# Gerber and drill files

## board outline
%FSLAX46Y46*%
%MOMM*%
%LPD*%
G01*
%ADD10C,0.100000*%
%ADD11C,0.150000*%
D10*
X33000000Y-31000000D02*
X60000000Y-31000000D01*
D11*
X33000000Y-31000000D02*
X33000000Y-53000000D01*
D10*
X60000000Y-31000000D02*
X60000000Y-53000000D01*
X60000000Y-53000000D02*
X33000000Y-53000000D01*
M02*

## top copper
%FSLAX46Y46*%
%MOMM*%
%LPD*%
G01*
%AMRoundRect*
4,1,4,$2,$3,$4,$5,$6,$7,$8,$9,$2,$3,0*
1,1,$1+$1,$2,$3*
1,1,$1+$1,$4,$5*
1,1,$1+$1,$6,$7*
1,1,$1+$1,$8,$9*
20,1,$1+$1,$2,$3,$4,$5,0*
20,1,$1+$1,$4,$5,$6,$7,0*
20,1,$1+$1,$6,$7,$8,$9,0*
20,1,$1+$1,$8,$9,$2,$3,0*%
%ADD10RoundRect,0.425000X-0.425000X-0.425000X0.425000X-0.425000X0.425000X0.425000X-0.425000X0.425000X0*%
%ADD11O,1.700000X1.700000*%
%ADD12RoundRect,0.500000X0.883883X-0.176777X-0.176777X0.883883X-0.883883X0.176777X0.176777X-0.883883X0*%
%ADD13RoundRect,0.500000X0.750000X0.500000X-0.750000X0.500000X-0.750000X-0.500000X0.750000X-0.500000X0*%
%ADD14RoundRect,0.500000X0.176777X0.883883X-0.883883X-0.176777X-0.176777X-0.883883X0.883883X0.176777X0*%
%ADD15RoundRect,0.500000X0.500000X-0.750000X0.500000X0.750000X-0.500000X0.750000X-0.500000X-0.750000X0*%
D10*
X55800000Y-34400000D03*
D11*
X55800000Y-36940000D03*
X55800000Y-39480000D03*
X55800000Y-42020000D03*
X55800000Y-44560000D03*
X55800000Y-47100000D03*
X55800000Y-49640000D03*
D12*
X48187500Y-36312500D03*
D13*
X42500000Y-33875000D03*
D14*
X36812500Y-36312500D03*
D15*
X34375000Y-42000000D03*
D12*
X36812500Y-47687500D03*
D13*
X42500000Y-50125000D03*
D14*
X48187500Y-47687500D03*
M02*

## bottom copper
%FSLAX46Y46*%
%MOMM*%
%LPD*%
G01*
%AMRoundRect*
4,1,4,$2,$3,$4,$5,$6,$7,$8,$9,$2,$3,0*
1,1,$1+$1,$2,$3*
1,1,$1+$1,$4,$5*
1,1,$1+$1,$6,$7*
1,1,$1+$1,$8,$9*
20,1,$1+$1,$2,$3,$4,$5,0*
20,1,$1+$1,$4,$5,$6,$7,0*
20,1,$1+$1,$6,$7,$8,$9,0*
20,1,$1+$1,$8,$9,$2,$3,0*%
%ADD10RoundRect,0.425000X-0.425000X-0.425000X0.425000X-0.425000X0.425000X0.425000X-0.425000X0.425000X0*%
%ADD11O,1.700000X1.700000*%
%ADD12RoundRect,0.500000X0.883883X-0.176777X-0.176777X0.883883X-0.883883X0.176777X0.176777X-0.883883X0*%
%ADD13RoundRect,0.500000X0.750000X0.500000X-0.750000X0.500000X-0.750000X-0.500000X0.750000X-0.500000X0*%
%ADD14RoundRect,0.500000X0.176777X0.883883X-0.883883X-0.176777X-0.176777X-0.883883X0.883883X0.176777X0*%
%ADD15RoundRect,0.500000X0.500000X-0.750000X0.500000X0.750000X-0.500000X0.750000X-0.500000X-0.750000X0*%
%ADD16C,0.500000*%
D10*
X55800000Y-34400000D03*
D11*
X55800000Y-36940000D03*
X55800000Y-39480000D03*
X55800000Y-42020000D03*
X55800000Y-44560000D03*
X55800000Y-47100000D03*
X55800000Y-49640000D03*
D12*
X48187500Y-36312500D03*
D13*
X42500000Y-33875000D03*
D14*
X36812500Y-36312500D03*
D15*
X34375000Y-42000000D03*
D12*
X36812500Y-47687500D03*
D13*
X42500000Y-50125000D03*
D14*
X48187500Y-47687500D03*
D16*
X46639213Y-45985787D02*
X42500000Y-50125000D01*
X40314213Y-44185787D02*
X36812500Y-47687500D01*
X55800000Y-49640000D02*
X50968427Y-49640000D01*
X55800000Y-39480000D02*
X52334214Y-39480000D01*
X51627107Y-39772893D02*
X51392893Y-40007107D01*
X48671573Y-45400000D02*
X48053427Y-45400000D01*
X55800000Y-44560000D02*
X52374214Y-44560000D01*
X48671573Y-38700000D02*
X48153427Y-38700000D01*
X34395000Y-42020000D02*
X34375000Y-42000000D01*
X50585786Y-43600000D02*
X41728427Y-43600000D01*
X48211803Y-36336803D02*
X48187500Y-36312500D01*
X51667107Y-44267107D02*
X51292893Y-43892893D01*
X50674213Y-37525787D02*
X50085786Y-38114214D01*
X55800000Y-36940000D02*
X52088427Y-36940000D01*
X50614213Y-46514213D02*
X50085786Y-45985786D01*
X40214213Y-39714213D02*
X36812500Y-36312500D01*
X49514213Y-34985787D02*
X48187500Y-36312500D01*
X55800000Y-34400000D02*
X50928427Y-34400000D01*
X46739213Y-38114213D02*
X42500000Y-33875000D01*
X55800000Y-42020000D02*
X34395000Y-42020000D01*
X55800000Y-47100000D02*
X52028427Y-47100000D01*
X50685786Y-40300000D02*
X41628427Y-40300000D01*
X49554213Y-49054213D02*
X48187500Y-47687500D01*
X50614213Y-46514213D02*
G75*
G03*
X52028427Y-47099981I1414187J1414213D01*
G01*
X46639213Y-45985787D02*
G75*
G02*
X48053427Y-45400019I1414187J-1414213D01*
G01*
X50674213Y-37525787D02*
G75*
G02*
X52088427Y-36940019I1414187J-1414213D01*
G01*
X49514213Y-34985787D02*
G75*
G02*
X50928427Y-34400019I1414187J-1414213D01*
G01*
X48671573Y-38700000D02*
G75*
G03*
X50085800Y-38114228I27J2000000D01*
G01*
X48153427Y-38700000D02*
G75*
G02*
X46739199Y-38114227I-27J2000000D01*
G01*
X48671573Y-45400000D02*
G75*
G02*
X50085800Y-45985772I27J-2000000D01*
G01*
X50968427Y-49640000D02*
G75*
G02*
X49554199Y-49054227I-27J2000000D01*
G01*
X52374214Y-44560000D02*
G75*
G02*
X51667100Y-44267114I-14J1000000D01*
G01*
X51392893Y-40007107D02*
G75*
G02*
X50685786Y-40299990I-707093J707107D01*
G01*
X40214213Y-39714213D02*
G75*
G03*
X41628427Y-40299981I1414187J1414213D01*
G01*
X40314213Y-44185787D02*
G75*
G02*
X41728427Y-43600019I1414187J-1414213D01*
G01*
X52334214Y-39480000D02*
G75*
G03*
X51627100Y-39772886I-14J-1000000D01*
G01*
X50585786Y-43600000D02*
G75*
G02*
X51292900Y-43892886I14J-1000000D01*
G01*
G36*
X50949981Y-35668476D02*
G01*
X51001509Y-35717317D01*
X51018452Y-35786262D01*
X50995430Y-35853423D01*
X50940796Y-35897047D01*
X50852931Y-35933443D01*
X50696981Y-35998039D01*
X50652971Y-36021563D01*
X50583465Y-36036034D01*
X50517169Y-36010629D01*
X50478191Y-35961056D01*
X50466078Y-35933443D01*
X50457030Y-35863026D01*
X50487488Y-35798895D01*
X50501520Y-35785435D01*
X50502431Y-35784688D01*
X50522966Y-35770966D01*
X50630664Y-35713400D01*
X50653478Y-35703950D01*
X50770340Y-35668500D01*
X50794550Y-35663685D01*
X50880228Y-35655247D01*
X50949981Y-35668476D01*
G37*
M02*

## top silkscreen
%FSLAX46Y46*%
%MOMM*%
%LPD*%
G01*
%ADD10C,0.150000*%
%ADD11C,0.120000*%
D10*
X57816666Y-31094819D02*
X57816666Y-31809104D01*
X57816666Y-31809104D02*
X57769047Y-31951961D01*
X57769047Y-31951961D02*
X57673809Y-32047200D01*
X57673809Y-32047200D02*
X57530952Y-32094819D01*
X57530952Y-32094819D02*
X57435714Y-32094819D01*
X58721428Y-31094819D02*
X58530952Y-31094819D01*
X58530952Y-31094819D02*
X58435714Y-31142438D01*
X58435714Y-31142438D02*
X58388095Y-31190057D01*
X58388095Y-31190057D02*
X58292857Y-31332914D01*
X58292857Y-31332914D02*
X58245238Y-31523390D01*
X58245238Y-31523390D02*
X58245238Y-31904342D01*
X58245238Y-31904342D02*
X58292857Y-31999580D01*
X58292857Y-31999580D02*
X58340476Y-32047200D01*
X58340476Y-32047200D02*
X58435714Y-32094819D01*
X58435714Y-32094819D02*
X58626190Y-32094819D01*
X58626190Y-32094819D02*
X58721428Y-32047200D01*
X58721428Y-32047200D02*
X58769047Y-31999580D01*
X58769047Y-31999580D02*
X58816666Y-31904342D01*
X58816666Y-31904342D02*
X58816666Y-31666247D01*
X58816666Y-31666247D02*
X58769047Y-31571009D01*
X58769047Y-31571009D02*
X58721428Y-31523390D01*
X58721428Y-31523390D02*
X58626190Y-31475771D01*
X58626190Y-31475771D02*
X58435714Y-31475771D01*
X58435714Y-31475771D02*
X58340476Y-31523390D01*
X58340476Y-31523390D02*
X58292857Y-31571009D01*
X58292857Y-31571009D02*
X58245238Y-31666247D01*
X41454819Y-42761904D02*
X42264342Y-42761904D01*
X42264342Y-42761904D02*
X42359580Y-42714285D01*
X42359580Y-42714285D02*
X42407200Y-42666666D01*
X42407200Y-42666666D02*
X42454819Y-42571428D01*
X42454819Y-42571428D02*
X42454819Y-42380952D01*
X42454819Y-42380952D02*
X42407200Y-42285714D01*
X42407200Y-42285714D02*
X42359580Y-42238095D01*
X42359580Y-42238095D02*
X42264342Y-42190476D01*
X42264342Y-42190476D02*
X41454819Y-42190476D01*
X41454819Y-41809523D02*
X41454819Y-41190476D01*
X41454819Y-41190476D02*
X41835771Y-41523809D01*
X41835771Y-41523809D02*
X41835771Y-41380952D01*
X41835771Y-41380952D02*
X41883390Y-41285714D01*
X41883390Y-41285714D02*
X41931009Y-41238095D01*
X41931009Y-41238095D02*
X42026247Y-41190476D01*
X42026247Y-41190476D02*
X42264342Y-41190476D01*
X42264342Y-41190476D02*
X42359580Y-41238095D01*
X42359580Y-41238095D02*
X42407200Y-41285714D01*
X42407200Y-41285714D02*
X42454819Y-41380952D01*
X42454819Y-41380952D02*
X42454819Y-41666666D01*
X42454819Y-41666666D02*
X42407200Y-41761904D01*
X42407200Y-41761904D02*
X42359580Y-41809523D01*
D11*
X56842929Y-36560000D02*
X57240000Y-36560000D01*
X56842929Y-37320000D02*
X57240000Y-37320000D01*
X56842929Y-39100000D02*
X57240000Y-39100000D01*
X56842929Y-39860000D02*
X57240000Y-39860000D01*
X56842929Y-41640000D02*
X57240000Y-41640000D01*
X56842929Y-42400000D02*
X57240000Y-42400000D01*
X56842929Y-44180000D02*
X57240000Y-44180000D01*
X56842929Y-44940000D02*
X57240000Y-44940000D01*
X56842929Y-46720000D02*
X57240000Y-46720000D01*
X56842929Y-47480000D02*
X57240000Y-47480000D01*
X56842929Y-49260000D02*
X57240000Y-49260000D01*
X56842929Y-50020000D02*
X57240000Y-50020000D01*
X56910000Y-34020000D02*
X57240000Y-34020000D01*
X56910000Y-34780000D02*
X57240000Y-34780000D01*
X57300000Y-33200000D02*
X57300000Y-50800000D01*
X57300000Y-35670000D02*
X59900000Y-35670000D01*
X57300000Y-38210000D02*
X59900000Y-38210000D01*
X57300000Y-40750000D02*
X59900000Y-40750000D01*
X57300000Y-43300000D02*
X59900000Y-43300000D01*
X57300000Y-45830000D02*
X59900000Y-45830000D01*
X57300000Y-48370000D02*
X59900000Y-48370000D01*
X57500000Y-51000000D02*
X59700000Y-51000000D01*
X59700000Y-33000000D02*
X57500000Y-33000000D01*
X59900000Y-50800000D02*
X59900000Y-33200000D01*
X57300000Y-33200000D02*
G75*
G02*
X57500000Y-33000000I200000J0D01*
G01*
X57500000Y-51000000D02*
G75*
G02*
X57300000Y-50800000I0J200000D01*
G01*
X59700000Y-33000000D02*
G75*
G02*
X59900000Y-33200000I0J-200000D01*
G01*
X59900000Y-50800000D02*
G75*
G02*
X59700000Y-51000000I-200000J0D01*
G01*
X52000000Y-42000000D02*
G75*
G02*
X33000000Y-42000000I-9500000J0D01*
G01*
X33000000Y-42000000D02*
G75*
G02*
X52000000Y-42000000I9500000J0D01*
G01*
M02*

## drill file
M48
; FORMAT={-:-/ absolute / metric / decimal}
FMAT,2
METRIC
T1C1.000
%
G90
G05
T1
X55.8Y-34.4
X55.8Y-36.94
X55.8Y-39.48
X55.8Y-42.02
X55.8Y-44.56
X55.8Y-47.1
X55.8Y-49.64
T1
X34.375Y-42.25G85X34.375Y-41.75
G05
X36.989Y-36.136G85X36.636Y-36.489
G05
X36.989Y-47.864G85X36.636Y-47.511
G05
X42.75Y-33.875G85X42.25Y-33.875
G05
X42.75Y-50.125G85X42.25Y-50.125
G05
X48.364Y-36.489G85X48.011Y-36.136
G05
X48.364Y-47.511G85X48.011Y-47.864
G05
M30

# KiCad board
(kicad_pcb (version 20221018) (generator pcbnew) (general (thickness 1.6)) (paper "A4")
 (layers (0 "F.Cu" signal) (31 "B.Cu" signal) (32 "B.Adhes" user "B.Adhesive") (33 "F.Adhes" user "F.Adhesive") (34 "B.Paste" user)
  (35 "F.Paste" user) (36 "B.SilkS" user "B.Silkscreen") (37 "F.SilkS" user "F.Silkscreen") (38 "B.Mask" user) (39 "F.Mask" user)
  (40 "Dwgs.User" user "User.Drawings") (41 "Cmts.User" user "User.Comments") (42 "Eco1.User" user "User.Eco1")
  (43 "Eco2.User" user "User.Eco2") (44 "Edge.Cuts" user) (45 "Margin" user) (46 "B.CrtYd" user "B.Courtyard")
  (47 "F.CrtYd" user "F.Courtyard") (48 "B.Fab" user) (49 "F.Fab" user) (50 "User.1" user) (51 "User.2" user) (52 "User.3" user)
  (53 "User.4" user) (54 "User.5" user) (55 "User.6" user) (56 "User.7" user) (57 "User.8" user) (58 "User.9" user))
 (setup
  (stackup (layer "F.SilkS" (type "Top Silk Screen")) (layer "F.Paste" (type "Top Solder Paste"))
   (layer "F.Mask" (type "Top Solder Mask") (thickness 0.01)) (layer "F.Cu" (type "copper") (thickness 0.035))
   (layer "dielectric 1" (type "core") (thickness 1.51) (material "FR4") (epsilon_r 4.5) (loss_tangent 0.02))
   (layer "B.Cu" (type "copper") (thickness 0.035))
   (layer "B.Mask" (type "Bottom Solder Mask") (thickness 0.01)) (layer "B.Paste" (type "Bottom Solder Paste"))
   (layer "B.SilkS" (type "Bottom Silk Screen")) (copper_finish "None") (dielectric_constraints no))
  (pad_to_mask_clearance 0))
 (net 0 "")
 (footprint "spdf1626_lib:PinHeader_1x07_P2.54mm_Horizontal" (layer "F.Cu") (at 55.8 34.4)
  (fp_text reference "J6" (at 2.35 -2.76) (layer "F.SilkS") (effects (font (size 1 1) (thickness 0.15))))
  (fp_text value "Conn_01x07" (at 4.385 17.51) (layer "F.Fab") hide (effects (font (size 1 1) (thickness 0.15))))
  (fp_line (start 1.042929 2.16) (end 1.44 2.16) (stroke (width 0.12) (type solid)) (layer "F.SilkS"))
  (fp_line (start 1.042929 2.92) (end 1.44 2.92) (stroke (width 0.12) (type solid)) (layer "F.SilkS"))
  (fp_line (start 1.042929 4.7) (end 1.44 4.7) (stroke (width 0.12) (type solid)) (layer "F.SilkS"))
  (fp_line (start 1.042929 5.46) (end 1.44 5.46) (stroke (width 0.12) (type solid)) (layer "F.SilkS"))
  (fp_line (start 1.042929 7.24) (end 1.44 7.24) (stroke (width 0.12) (type solid)) (layer "F.SilkS"))
  (fp_line (start 1.042929 8) (end 1.44 8) (stroke (width 0.12) (type solid)) (layer "F.SilkS"))
  (fp_line (start 1.042929 9.78) (end 1.44 9.78) (stroke (width 0.12) (type solid)) (layer "F.SilkS"))
  (fp_line (start 1.042929 10.54) (end 1.44 10.54) (stroke (width 0.12) (type solid)) (layer "F.SilkS"))
  (fp_line (start 1.042929 12.32) (end 1.44 12.32) (stroke (width 0.12) (type solid)) (layer "F.SilkS"))
  (fp_line (start 1.042929 13.08) (end 1.44 13.08) (stroke (width 0.12) (type solid)) (layer "F.SilkS"))
  (fp_line (start 1.042929 14.86) (end 1.44 14.86) (stroke (width 0.12) (type solid)) (layer "F.SilkS"))
  (fp_line (start 1.042929 15.62) (end 1.44 15.62) (stroke (width 0.12) (type solid)) (layer "F.SilkS"))
  (fp_line (start 1.11 -0.38) (end 1.44 -0.38) (stroke (width 0.12) (type solid)) (layer "F.SilkS"))
  (fp_line (start 1.11 0.38) (end 1.44 0.38) (stroke (width 0.12) (type solid)) (layer "F.SilkS"))
  (fp_line (start 1.5 -1.2) (end 1.5 16.4) (stroke (width 0.12) (type solid)) (layer "F.SilkS"))
  (fp_line (start 1.5 1.27) (end 4.1 1.27) (stroke (width 0.12) (type solid)) (layer "F.SilkS"))
  (fp_line (start 1.5 3.81) (end 4.1 3.81) (stroke (width 0.12) (type solid)) (layer "F.SilkS"))
  (fp_line (start 1.5 6.35) (end 4.1 6.35) (stroke (width 0.12) (type solid)) (layer "F.SilkS"))
  (fp_line (start 1.5 8.9) (end 4.1 8.9) (stroke (width 0.12) (type solid)) (layer "F.SilkS"))
  (fp_line (start 1.5 11.43) (end 4.1 11.43) (stroke (width 0.12) (type solid)) (layer "F.SilkS"))
  (fp_line (start 1.5 13.97) (end 4.1 13.97) (stroke (width 0.12) (type solid)) (layer "F.SilkS"))
  (fp_line (start 1.7 16.6) (end 3.9 16.6) (stroke (width 0.12) (type solid)) (layer "F.SilkS"))
  (fp_line (start 3.9 -1.4) (end 1.7 -1.4) (stroke (width 0.12) (type solid)) (layer "F.SilkS"))
  (fp_line (start 4.1 16.4) (end 4.1 -1.2) (stroke (width 0.12) (type solid)) (layer "F.SilkS"))
  (fp_arc (start 1.5 -1.2) (mid 1.558579 -1.341421) (end 1.7 -1.4) (stroke (width 0.12) (type solid)) (layer "F.SilkS"))
  (fp_arc (start 1.7 16.6) (mid 1.558579 16.541421) (end 1.5 16.4) (stroke (width 0.12) (type solid)) (layer "F.SilkS"))
  (fp_arc (start 3.9 -1.4) (mid 4.041421 -1.341421) (end 4.1 -1.2) (stroke (width 0.12) (type solid)) (layer "F.SilkS"))
  (fp_arc (start 4.1 16.4) (mid 4.041421 16.541421) (end 3.9 16.6) (stroke (width 0.12) (type solid)) (layer "F.SilkS"))
  (pad "1" thru_hole roundrect (at 0 0) (size 1.7 1.7) (drill 1) (layers "*.Cu" "*.Mask") (roundrect_rratio 0.25))
  (pad "2" thru_hole oval (at 0 2.54) (size 1.7 1.7) (drill 1) (layers "*.Cu" "*.Mask"))
  (pad "3" thru_hole oval (at 0 5.08) (size 1.7 1.7) (drill 1) (layers "*.Cu" "*.Mask"))
  (pad "4" thru_hole oval (at 0 7.62) (size 1.7 1.7) (drill 1) (layers "*.Cu" "*.Mask"))
  (pad "5" thru_hole oval (at 0 10.16) (size 1.7 1.7) (drill 1) (layers "*.Cu" "*.Mask"))
  (pad "6" thru_hole oval (at 0 12.7) (size 1.7 1.7) (drill 1) (layers "*.Cu" "*.Mask"))
  (pad "7" thru_hole oval (at 0 15.24) (size 1.7 1.7) (drill 1) (layers "*.Cu" "*.Mask")))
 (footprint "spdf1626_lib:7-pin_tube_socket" (layer "F.Cu") (at 42.5 42 90)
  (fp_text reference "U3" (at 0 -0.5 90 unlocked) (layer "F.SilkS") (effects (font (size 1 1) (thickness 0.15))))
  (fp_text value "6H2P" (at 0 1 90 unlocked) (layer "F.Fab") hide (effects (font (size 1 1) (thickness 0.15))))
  (fp_circle (center 0 0) (end 9.5 0) (stroke (width 0.12) (type solid)) (fill none) (layer "F.SilkS"))
  (pad "1" thru_hole roundrect (at 5.6875 5.6875 135) (size 2.5 2) (drill oval 1.5 1) (layers "*.Cu" "*.Mask") (roundrect_rratio 0.25))
  (pad "2" thru_hole roundrect (at 8.125 0 180) (size 2.5 2) (drill oval 1.5 1) (layers "*.Cu" "*.Mask") (roundrect_rratio 0.25))
  (pad "3" thru_hole roundrect (at 5.6875 -5.6875 225) (size 2.5 2) (drill oval 1.5 1) (layers "*.Cu" "*.Mask") (roundrect_rratio 0.25))
  (pad "4" thru_hole roundrect (at 0 -8.125 90) (size 2.5 2) (drill oval 1.5 1) (layers "*.Cu" "*.Mask") (roundrect_rratio 0.25))
  (pad "5" thru_hole roundrect (at -5.6875 -5.6875 135) (size 2.5 2) (drill oval 1.5 1) (layers "*.Cu" "*.Mask") (roundrect_rratio 0.25))
  (pad "6" thru_hole roundrect (at -8.125 0 180) (size 2.5 2) (drill oval 1.5 1) (layers "*.Cu" "*.Mask") (roundrect_rratio 0.25))
  (pad "7" thru_hole roundrect (at -5.6875 5.6875 225) (size 2.5 2) (drill oval 1.5 1) (layers "*.Cu" "*.Mask") (roundrect_rratio 0.25)))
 (gr_line (start 33 31) (end 60 31) (stroke (width 0.1) (type default)) (layer "Edge.Cuts"))
 (gr_line (start 33 31) (end 33 53) (stroke (width 0.15) (type solid)) (layer "Edge.Cuts"))
 (gr_line (start 60 31) (end 60 53) (stroke (width 0.1) (type default)) (layer "Edge.Cuts"))
 (gr_line (start 60 53) (end 33 53) (stroke (width 0.1) (type default)) (layer "Edge.Cuts"))
 (segment (start 46.639213 45.985787) (end 42.5 50.125) (width 0.5) (layer "B.Cu") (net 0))
 (segment (start 40.314213 44.185787) (end 36.8125 47.6875) (width 0.5) (layer "B.Cu") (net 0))
 (segment (start 55.8 49.64) (end 50.968427 49.64) (width 0.5) (layer "B.Cu") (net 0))
 (segment (start 55.8 39.48) (end 52.334214 39.48) (width 0.5) (layer "B.Cu") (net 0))
 (segment (start 51.627107 39.772893) (end 51.392893 40.007107) (width 0.5) (layer "B.Cu") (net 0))
 (segment (start 48.671573 45.4) (end 48.053427 45.4) (width 0.5) (layer "B.Cu") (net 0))
 (segment (start 55.8 44.56) (end 52.374214 44.56) (width 0.5) (layer "B.Cu") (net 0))
 (segment (start 48.671573 38.7) (end 48.153427 38.7) (width 0.5) (layer "B.Cu") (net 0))
 (segment (start 34.395 42.02) (end 34.375 42) (width 0.5) (layer "B.Cu") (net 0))
 (segment (start 50.585786 43.6) (end 41.728427 43.6) (width 0.5) (layer "B.Cu") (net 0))
 (segment (start 48.211803 36.336803) (end 48.1875 36.3125) (width 0.5) (layer "B.Cu") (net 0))
 (segment (start 51.667107 44.267107) (end 51.292893 43.892893) (width 0.5) (layer "B.Cu") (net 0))
 (segment (start 50.674213 37.525787) (end 50.085786 38.114214) (width 0.5) (layer "B.Cu") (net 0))
 (segment (start 55.8 36.94) (end 52.088427 36.94) (width 0.5) (layer "B.Cu") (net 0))
 (segment (start 50.614213 46.514213) (end 50.085786 45.985786) (width 0.5) (layer "B.Cu") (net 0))
 (segment (start 40.214213 39.714213) (end 36.8125 36.3125) (width 0.5) (layer "B.Cu") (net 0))
 (segment (start 49.514213 34.985787) (end 48.1875 36.3125) (width 0.5) (layer "B.Cu") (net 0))
 (segment (start 55.8 34.4) (end 50.928427 34.4) (width 0.5) (layer "B.Cu") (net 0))
 (segment (start 46.739213 38.114213) (end 42.5 33.875) (width 0.5) (layer "B.Cu") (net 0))
 (segment (start 55.8 42.02) (end 34.395 42.02) (width 0.5) (layer "B.Cu") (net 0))
 (segment (start 55.8 47.1) (end 52.028427 47.1) (width 0.5) (layer "B.Cu") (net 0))
 (segment (start 50.685786 40.3) (end 41.628427 40.3) (width 0.5) (layer "B.Cu") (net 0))
 (segment (start 49.554213 49.054213) (end 48.1875 47.6875) (width 0.5) (layer "B.Cu") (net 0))
 (arc (start 50.614213 46.514213) (mid 51.26306 46.947759) (end 52.028427 47.1) (width 0.5) (layer "B.Cu") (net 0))
 (arc (start 46.639213 45.985787) (mid 47.28806 45.552241) (end 48.053427 45.4) (width 0.5) (layer "B.Cu") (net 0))
 (arc (start 50.674213 37.525787) (mid 51.32306 37.092241) (end 52.088427 36.94) (width 0.5) (layer "B.Cu") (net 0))
 (arc (start 49.514213 34.985787) (mid 50.16306 34.552241) (end 50.928427 34.4) (width 0.5) (layer "B.Cu") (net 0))
 (arc (start 48.671573 38.7) (mid 49.43694 38.547759) (end 50.085786 38.114214) (width 0.5) (layer "B.Cu") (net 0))
 (arc (start 48.153427 38.7) (mid 47.38806 38.547759) (end 46.739213 38.114213) (width 0.5) (layer "B.Cu") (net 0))
 (arc (start 48.671573 45.4) (mid 49.43694 45.552241) (end 50.085786 45.985786) (width 0.5) (layer "B.Cu") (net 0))
 (arc (start 50.968427 49.64) (mid 50.20306 49.487759) (end 49.554213 49.054213) (width 0.5) (layer "B.Cu") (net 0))
 (arc (start 52.374214 44.56) (mid 51.991531 44.48388) (end 51.667107 44.267107) (width 0.5) (layer "B.Cu") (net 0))
 (arc (start 51.392893 40.007107) (mid 51.06847 40.22388) (end 50.685786 40.3) (width 0.5) (layer "B.Cu") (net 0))
 (arc (start 40.214213 39.714213) (mid 40.86306 40.147759) (end 41.628427 40.3) (width 0.5) (layer "B.Cu") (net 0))
 (arc (start 40.314213 44.185787) (mid 40.96306 43.752241) (end 41.728427 43.6) (width 0.5) (layer "B.Cu") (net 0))
 (arc (start 52.334214 39.48) (mid 51.951531 39.55612) (end 51.627107 39.772893) (width 0.5) (layer "B.Cu") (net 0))
 (arc (start 50.585786 43.6) (mid 50.968469 43.67612) (end 51.292893 43.892893) (width 0.5) (layer "B.Cu") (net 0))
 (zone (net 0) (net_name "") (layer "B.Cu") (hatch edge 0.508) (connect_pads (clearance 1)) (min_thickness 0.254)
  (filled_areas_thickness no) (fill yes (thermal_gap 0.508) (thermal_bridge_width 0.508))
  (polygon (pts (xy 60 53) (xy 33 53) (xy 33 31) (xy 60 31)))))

